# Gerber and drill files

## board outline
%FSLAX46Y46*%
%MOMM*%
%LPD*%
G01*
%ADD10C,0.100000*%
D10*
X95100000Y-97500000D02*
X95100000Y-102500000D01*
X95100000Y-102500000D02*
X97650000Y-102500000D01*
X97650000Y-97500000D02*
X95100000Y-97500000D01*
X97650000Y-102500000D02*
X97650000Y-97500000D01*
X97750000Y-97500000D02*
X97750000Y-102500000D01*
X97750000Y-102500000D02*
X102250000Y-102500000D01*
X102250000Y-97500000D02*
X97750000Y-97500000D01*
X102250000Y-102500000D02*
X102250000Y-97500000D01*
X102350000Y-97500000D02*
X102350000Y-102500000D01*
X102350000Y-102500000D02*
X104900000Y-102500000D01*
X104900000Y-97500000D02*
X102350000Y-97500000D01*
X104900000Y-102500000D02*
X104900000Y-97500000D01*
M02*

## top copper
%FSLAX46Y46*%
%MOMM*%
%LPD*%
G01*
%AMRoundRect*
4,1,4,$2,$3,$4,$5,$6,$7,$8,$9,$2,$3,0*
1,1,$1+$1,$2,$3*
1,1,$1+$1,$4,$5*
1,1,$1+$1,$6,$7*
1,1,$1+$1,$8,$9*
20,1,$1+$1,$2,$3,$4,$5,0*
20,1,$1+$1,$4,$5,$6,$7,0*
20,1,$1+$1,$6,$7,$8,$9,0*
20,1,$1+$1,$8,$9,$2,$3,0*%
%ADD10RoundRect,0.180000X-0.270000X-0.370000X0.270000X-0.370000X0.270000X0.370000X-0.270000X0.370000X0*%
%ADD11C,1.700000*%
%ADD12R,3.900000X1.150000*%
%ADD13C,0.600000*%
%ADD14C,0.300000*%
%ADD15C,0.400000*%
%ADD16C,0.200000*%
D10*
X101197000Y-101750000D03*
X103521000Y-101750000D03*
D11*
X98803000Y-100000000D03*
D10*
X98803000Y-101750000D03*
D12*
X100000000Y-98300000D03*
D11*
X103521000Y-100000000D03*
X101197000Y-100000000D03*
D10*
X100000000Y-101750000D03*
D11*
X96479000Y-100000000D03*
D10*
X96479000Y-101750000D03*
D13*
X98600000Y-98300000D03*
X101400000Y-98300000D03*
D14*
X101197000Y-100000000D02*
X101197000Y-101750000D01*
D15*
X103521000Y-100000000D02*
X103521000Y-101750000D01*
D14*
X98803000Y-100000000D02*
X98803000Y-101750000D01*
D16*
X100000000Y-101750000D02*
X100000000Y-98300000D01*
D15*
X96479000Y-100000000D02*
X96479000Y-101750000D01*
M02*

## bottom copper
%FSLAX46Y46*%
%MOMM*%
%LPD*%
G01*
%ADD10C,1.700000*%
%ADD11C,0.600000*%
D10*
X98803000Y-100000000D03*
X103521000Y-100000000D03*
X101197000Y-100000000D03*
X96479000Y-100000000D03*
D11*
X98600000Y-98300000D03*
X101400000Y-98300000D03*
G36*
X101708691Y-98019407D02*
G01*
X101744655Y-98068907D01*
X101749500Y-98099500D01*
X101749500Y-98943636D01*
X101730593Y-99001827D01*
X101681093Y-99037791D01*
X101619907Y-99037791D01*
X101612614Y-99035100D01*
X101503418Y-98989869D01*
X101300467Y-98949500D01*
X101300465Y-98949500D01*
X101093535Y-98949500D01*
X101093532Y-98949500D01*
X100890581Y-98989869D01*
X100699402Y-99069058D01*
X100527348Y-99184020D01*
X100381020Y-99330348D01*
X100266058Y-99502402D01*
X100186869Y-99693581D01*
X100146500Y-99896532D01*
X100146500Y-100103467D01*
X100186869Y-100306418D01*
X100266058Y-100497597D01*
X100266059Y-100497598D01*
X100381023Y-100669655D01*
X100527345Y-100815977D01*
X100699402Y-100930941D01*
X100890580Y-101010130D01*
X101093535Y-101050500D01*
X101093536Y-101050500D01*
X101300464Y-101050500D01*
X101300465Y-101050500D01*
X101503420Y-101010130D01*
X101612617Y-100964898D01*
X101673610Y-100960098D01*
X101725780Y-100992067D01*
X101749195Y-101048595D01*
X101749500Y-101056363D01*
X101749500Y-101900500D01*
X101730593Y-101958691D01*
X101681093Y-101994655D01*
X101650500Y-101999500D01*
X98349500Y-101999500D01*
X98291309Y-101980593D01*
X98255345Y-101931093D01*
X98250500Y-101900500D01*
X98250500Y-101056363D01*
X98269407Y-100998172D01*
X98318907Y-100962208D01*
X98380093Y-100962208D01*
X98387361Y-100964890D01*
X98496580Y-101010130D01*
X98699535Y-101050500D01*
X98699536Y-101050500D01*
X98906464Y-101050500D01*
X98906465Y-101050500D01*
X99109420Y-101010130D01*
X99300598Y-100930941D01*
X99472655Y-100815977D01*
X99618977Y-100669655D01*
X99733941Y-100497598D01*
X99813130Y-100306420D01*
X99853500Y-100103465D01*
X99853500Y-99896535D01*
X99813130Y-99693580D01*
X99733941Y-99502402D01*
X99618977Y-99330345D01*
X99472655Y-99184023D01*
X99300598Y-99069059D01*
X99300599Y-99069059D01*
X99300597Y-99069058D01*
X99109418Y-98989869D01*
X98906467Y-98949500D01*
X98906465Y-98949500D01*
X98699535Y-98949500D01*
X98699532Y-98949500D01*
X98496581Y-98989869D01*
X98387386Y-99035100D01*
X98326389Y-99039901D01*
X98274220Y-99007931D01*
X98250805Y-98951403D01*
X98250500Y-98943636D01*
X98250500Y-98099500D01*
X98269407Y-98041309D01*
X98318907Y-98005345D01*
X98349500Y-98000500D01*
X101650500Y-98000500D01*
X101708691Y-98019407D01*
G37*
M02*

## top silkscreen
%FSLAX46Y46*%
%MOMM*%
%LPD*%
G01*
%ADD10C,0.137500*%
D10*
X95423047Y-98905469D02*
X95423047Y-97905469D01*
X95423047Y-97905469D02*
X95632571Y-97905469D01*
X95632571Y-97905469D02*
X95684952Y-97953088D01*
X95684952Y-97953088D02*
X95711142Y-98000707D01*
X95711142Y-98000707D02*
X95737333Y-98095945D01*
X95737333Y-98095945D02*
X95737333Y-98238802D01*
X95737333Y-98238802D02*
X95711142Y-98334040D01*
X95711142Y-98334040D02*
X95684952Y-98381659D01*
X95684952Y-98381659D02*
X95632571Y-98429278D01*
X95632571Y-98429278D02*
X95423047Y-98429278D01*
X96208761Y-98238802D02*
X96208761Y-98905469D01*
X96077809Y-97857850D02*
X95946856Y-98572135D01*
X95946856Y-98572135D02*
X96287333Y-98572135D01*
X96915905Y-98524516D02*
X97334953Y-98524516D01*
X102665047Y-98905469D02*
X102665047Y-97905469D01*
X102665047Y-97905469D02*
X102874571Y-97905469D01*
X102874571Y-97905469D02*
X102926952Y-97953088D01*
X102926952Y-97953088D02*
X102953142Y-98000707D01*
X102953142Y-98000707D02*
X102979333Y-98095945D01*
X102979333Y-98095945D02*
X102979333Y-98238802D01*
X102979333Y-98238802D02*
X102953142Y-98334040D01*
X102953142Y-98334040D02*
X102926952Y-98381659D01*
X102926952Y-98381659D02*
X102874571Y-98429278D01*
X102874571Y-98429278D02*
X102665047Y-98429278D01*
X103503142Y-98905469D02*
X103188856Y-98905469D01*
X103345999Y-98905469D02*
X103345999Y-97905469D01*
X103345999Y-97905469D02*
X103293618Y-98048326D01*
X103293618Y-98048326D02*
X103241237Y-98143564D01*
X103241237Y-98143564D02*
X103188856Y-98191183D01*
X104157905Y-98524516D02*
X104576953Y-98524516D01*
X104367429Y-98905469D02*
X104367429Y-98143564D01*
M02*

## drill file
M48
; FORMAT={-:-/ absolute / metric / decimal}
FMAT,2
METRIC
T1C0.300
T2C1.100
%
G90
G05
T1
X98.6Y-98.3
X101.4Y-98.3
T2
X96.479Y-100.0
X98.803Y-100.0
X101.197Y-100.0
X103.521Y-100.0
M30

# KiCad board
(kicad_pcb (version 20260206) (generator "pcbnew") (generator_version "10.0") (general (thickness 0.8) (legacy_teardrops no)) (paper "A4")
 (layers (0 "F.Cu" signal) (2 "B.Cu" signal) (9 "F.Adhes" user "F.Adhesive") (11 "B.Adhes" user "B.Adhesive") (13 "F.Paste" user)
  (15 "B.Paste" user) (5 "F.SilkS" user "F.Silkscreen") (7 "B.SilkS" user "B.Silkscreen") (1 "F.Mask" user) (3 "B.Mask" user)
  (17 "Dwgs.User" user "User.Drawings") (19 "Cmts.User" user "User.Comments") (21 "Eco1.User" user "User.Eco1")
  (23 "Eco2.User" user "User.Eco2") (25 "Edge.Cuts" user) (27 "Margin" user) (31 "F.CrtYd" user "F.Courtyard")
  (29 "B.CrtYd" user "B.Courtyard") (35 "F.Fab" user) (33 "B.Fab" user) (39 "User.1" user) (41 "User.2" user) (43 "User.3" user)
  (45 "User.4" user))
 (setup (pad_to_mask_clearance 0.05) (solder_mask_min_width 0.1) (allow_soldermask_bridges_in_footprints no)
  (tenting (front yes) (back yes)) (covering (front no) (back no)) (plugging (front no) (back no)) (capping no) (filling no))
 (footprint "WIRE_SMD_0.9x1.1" (layer "F.Cu") (at 101.197 101.75)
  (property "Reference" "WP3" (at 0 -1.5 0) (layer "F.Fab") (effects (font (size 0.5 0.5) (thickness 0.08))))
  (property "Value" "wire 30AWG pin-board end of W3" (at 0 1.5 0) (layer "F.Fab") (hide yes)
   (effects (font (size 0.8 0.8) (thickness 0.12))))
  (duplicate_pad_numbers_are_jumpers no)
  (pad "1" smd roundrect (at 0 0) (size 0.9 1.1) (layers "F.Cu" "F.Mask") (roundrect_rratio 0.2) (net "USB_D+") (thermal_bridge_angle 45)))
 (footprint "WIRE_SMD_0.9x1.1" (layer "F.Cu") (at 103.521 101.75)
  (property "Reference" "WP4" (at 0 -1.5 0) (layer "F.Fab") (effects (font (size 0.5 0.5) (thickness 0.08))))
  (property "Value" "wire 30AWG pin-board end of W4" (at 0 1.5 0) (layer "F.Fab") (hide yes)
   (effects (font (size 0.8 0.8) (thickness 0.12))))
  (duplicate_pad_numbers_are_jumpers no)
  (pad "1" smd roundrect (at 0 0) (size 0.9 1.1) (layers "F.Cu" "F.Mask") (roundrect_rratio 0.2) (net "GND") (thermal_bridge_angle 45)))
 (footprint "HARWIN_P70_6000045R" (layer "F.Cu") (at 98.803 100)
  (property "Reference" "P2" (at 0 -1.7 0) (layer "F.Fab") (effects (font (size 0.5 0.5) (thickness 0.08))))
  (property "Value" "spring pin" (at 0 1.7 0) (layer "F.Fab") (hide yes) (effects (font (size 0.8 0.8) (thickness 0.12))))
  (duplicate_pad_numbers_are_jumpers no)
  (pad "1" thru_hole circle (at 0 0) (size 1.7 1.7) (drill 1.1) (layers "*.Cu" "*.Mask") (remove_unused_layers no) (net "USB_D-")))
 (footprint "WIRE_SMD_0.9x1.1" (layer "F.Cu") (at 98.803 101.75)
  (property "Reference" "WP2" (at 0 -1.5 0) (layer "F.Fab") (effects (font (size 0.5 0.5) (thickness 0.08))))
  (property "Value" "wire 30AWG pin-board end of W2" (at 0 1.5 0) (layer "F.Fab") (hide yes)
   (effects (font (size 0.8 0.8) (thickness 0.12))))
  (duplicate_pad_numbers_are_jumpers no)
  (pad "1" smd roundrect (at 0 0) (size 0.9 1.1) (layers "F.Cu" "F.Mask") (roundrect_rratio 0.2) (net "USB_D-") (thermal_bridge_angle 45)))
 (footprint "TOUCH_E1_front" (layer "F.Cu") (at 100 98.3)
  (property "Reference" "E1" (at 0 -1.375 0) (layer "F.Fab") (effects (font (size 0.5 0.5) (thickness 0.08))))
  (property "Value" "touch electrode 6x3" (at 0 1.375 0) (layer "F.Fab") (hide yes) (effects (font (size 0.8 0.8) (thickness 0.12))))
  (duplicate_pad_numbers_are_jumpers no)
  (pad "1" smd rect (at 0 0) (size 3.9 1.15) (layers "F.Cu" "F.Mask") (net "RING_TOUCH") (thermal_bridge_angle 45)))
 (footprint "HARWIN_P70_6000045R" (layer "F.Cu") (at 103.521 100)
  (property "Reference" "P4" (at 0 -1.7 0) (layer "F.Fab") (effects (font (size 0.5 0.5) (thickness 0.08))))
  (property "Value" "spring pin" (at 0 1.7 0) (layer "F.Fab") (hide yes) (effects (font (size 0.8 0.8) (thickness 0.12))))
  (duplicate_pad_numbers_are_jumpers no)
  (pad "1" thru_hole circle (at 0 0) (size 1.7 1.7) (drill 1.1) (layers "*.Cu" "*.Mask") (remove_unused_layers no) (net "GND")))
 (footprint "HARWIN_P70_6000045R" (layer "F.Cu") (at 101.197 100)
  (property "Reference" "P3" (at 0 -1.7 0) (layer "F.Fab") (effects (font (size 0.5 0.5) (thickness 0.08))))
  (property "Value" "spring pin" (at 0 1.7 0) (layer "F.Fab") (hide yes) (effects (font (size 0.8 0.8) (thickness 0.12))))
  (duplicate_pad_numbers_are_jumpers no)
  (pad "1" thru_hole circle (at 0 0) (size 1.7 1.7) (drill 1.1) (layers "*.Cu" "*.Mask") (remove_unused_layers no) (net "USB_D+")))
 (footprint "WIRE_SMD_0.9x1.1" (layer "F.Cu") (at 100 101.75)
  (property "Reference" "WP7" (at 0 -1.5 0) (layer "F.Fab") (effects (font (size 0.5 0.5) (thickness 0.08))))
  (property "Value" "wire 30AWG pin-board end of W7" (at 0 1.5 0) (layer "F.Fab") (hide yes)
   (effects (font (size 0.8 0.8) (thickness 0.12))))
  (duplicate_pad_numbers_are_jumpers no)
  (pad "1" smd roundrect (at 0 0) (size 0.9 1.1) (layers "F.Cu" "F.Mask") (roundrect_rratio 0.2) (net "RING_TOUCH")
   (thermal_bridge_angle 45)))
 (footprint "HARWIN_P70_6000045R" (layer "F.Cu") (at 96.479 100)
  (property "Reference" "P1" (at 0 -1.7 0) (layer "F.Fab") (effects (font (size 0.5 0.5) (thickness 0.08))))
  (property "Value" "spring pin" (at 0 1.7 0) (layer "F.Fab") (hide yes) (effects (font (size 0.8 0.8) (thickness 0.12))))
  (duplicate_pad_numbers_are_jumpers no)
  (pad "1" thru_hole circle (at 0 0) (size 1.7 1.7) (drill 1.1) (layers "*.Cu" "*.Mask") (remove_unused_layers no) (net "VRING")))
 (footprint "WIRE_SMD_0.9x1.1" (layer "F.Cu") (at 96.479 101.75)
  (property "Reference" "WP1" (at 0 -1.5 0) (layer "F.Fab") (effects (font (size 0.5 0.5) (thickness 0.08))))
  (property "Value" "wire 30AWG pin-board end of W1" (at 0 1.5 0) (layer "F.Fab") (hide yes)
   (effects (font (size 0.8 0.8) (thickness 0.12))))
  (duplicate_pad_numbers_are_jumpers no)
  (pad "1" smd roundrect (at 0 0) (size 0.9 1.1) (layers "F.Cu" "F.Mask") (roundrect_rratio 0.2) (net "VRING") (thermal_bridge_angle 45)))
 (gr_line (start 95.1 97.5) (end 95.1 102.5) (stroke (width 0.1) (type default)) (layer "Edge.Cuts"))
 (gr_line (start 95.1 102.5) (end 97.65 102.5) (stroke (width 0.1) (type default)) (layer "Edge.Cuts"))
 (gr_line (start 97.65 97.5) (end 95.1 97.5) (stroke (width 0.1) (type default)) (layer "Edge.Cuts"))
 (gr_line (start 97.65 102.5) (end 97.65 97.5) (stroke (width 0.1) (type default)) (layer "Edge.Cuts"))
 (gr_line (start 97.75 97.5) (end 97.75 102.5) (stroke (width 0.1) (type default)) (layer "Edge.Cuts"))
 (gr_line (start 97.75 102.5) (end 102.25 102.5) (stroke (width 0.1) (type default)) (layer "Edge.Cuts"))
 (gr_line (start 102.25 97.5) (end 97.75 97.5) (stroke (width 0.1) (type default)) (layer "Edge.Cuts"))
 (gr_line (start 102.25 102.5) (end 102.25 97.5) (stroke (width 0.1) (type default)) (layer "Edge.Cuts"))
 (gr_line (start 102.35 97.5) (end 102.35 102.5) (stroke (width 0.1) (type default)) (layer "Edge.Cuts"))
 (gr_line (start 102.35 102.5) (end 104.9 102.5) (stroke (width 0.1) (type default)) (layer "Edge.Cuts"))
 (gr_line (start 104.9 97.5) (end 102.35 97.5) (stroke (width 0.1) (type default)) (layer "Edge.Cuts"))
 (gr_line (start 104.9 102.5) (end 104.9 97.5) (stroke (width 0.1) (type default)) (layer "Edge.Cuts"))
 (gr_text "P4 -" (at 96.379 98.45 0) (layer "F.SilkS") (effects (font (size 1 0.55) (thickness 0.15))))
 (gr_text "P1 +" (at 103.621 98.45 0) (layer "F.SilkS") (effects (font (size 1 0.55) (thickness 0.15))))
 (segment (start 101.197 100) (end 101.197 101.75) (width 0.3) (layer "F.Cu") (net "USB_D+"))
 (segment (start 103.521 100) (end 103.521 101.75) (width 0.4) (layer "F.Cu") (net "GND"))
 (segment (start 98.803 100) (end 98.803 101.75) (width 0.3) (layer "F.Cu") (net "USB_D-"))
 (segment (start 100 101.75) (end 100 98.3) (width 0.2) (layer "F.Cu") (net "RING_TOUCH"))
 (via (at 98.6 98.3) (size 0.6) (drill 0.3) (layers "F.Cu" "B.Cu") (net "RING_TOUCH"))
 (via (at 101.4 98.3) (size 0.6) (drill 0.3) (layers "F.Cu" "B.Cu") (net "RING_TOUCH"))
 (segment (start 96.479 100) (end 96.479 101.75) (width 0.4) (layer "F.Cu") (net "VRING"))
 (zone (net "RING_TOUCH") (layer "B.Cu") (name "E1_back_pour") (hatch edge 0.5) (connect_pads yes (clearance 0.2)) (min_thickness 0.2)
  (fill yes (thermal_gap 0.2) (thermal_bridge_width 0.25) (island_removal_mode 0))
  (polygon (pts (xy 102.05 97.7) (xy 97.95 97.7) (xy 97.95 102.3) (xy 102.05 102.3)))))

